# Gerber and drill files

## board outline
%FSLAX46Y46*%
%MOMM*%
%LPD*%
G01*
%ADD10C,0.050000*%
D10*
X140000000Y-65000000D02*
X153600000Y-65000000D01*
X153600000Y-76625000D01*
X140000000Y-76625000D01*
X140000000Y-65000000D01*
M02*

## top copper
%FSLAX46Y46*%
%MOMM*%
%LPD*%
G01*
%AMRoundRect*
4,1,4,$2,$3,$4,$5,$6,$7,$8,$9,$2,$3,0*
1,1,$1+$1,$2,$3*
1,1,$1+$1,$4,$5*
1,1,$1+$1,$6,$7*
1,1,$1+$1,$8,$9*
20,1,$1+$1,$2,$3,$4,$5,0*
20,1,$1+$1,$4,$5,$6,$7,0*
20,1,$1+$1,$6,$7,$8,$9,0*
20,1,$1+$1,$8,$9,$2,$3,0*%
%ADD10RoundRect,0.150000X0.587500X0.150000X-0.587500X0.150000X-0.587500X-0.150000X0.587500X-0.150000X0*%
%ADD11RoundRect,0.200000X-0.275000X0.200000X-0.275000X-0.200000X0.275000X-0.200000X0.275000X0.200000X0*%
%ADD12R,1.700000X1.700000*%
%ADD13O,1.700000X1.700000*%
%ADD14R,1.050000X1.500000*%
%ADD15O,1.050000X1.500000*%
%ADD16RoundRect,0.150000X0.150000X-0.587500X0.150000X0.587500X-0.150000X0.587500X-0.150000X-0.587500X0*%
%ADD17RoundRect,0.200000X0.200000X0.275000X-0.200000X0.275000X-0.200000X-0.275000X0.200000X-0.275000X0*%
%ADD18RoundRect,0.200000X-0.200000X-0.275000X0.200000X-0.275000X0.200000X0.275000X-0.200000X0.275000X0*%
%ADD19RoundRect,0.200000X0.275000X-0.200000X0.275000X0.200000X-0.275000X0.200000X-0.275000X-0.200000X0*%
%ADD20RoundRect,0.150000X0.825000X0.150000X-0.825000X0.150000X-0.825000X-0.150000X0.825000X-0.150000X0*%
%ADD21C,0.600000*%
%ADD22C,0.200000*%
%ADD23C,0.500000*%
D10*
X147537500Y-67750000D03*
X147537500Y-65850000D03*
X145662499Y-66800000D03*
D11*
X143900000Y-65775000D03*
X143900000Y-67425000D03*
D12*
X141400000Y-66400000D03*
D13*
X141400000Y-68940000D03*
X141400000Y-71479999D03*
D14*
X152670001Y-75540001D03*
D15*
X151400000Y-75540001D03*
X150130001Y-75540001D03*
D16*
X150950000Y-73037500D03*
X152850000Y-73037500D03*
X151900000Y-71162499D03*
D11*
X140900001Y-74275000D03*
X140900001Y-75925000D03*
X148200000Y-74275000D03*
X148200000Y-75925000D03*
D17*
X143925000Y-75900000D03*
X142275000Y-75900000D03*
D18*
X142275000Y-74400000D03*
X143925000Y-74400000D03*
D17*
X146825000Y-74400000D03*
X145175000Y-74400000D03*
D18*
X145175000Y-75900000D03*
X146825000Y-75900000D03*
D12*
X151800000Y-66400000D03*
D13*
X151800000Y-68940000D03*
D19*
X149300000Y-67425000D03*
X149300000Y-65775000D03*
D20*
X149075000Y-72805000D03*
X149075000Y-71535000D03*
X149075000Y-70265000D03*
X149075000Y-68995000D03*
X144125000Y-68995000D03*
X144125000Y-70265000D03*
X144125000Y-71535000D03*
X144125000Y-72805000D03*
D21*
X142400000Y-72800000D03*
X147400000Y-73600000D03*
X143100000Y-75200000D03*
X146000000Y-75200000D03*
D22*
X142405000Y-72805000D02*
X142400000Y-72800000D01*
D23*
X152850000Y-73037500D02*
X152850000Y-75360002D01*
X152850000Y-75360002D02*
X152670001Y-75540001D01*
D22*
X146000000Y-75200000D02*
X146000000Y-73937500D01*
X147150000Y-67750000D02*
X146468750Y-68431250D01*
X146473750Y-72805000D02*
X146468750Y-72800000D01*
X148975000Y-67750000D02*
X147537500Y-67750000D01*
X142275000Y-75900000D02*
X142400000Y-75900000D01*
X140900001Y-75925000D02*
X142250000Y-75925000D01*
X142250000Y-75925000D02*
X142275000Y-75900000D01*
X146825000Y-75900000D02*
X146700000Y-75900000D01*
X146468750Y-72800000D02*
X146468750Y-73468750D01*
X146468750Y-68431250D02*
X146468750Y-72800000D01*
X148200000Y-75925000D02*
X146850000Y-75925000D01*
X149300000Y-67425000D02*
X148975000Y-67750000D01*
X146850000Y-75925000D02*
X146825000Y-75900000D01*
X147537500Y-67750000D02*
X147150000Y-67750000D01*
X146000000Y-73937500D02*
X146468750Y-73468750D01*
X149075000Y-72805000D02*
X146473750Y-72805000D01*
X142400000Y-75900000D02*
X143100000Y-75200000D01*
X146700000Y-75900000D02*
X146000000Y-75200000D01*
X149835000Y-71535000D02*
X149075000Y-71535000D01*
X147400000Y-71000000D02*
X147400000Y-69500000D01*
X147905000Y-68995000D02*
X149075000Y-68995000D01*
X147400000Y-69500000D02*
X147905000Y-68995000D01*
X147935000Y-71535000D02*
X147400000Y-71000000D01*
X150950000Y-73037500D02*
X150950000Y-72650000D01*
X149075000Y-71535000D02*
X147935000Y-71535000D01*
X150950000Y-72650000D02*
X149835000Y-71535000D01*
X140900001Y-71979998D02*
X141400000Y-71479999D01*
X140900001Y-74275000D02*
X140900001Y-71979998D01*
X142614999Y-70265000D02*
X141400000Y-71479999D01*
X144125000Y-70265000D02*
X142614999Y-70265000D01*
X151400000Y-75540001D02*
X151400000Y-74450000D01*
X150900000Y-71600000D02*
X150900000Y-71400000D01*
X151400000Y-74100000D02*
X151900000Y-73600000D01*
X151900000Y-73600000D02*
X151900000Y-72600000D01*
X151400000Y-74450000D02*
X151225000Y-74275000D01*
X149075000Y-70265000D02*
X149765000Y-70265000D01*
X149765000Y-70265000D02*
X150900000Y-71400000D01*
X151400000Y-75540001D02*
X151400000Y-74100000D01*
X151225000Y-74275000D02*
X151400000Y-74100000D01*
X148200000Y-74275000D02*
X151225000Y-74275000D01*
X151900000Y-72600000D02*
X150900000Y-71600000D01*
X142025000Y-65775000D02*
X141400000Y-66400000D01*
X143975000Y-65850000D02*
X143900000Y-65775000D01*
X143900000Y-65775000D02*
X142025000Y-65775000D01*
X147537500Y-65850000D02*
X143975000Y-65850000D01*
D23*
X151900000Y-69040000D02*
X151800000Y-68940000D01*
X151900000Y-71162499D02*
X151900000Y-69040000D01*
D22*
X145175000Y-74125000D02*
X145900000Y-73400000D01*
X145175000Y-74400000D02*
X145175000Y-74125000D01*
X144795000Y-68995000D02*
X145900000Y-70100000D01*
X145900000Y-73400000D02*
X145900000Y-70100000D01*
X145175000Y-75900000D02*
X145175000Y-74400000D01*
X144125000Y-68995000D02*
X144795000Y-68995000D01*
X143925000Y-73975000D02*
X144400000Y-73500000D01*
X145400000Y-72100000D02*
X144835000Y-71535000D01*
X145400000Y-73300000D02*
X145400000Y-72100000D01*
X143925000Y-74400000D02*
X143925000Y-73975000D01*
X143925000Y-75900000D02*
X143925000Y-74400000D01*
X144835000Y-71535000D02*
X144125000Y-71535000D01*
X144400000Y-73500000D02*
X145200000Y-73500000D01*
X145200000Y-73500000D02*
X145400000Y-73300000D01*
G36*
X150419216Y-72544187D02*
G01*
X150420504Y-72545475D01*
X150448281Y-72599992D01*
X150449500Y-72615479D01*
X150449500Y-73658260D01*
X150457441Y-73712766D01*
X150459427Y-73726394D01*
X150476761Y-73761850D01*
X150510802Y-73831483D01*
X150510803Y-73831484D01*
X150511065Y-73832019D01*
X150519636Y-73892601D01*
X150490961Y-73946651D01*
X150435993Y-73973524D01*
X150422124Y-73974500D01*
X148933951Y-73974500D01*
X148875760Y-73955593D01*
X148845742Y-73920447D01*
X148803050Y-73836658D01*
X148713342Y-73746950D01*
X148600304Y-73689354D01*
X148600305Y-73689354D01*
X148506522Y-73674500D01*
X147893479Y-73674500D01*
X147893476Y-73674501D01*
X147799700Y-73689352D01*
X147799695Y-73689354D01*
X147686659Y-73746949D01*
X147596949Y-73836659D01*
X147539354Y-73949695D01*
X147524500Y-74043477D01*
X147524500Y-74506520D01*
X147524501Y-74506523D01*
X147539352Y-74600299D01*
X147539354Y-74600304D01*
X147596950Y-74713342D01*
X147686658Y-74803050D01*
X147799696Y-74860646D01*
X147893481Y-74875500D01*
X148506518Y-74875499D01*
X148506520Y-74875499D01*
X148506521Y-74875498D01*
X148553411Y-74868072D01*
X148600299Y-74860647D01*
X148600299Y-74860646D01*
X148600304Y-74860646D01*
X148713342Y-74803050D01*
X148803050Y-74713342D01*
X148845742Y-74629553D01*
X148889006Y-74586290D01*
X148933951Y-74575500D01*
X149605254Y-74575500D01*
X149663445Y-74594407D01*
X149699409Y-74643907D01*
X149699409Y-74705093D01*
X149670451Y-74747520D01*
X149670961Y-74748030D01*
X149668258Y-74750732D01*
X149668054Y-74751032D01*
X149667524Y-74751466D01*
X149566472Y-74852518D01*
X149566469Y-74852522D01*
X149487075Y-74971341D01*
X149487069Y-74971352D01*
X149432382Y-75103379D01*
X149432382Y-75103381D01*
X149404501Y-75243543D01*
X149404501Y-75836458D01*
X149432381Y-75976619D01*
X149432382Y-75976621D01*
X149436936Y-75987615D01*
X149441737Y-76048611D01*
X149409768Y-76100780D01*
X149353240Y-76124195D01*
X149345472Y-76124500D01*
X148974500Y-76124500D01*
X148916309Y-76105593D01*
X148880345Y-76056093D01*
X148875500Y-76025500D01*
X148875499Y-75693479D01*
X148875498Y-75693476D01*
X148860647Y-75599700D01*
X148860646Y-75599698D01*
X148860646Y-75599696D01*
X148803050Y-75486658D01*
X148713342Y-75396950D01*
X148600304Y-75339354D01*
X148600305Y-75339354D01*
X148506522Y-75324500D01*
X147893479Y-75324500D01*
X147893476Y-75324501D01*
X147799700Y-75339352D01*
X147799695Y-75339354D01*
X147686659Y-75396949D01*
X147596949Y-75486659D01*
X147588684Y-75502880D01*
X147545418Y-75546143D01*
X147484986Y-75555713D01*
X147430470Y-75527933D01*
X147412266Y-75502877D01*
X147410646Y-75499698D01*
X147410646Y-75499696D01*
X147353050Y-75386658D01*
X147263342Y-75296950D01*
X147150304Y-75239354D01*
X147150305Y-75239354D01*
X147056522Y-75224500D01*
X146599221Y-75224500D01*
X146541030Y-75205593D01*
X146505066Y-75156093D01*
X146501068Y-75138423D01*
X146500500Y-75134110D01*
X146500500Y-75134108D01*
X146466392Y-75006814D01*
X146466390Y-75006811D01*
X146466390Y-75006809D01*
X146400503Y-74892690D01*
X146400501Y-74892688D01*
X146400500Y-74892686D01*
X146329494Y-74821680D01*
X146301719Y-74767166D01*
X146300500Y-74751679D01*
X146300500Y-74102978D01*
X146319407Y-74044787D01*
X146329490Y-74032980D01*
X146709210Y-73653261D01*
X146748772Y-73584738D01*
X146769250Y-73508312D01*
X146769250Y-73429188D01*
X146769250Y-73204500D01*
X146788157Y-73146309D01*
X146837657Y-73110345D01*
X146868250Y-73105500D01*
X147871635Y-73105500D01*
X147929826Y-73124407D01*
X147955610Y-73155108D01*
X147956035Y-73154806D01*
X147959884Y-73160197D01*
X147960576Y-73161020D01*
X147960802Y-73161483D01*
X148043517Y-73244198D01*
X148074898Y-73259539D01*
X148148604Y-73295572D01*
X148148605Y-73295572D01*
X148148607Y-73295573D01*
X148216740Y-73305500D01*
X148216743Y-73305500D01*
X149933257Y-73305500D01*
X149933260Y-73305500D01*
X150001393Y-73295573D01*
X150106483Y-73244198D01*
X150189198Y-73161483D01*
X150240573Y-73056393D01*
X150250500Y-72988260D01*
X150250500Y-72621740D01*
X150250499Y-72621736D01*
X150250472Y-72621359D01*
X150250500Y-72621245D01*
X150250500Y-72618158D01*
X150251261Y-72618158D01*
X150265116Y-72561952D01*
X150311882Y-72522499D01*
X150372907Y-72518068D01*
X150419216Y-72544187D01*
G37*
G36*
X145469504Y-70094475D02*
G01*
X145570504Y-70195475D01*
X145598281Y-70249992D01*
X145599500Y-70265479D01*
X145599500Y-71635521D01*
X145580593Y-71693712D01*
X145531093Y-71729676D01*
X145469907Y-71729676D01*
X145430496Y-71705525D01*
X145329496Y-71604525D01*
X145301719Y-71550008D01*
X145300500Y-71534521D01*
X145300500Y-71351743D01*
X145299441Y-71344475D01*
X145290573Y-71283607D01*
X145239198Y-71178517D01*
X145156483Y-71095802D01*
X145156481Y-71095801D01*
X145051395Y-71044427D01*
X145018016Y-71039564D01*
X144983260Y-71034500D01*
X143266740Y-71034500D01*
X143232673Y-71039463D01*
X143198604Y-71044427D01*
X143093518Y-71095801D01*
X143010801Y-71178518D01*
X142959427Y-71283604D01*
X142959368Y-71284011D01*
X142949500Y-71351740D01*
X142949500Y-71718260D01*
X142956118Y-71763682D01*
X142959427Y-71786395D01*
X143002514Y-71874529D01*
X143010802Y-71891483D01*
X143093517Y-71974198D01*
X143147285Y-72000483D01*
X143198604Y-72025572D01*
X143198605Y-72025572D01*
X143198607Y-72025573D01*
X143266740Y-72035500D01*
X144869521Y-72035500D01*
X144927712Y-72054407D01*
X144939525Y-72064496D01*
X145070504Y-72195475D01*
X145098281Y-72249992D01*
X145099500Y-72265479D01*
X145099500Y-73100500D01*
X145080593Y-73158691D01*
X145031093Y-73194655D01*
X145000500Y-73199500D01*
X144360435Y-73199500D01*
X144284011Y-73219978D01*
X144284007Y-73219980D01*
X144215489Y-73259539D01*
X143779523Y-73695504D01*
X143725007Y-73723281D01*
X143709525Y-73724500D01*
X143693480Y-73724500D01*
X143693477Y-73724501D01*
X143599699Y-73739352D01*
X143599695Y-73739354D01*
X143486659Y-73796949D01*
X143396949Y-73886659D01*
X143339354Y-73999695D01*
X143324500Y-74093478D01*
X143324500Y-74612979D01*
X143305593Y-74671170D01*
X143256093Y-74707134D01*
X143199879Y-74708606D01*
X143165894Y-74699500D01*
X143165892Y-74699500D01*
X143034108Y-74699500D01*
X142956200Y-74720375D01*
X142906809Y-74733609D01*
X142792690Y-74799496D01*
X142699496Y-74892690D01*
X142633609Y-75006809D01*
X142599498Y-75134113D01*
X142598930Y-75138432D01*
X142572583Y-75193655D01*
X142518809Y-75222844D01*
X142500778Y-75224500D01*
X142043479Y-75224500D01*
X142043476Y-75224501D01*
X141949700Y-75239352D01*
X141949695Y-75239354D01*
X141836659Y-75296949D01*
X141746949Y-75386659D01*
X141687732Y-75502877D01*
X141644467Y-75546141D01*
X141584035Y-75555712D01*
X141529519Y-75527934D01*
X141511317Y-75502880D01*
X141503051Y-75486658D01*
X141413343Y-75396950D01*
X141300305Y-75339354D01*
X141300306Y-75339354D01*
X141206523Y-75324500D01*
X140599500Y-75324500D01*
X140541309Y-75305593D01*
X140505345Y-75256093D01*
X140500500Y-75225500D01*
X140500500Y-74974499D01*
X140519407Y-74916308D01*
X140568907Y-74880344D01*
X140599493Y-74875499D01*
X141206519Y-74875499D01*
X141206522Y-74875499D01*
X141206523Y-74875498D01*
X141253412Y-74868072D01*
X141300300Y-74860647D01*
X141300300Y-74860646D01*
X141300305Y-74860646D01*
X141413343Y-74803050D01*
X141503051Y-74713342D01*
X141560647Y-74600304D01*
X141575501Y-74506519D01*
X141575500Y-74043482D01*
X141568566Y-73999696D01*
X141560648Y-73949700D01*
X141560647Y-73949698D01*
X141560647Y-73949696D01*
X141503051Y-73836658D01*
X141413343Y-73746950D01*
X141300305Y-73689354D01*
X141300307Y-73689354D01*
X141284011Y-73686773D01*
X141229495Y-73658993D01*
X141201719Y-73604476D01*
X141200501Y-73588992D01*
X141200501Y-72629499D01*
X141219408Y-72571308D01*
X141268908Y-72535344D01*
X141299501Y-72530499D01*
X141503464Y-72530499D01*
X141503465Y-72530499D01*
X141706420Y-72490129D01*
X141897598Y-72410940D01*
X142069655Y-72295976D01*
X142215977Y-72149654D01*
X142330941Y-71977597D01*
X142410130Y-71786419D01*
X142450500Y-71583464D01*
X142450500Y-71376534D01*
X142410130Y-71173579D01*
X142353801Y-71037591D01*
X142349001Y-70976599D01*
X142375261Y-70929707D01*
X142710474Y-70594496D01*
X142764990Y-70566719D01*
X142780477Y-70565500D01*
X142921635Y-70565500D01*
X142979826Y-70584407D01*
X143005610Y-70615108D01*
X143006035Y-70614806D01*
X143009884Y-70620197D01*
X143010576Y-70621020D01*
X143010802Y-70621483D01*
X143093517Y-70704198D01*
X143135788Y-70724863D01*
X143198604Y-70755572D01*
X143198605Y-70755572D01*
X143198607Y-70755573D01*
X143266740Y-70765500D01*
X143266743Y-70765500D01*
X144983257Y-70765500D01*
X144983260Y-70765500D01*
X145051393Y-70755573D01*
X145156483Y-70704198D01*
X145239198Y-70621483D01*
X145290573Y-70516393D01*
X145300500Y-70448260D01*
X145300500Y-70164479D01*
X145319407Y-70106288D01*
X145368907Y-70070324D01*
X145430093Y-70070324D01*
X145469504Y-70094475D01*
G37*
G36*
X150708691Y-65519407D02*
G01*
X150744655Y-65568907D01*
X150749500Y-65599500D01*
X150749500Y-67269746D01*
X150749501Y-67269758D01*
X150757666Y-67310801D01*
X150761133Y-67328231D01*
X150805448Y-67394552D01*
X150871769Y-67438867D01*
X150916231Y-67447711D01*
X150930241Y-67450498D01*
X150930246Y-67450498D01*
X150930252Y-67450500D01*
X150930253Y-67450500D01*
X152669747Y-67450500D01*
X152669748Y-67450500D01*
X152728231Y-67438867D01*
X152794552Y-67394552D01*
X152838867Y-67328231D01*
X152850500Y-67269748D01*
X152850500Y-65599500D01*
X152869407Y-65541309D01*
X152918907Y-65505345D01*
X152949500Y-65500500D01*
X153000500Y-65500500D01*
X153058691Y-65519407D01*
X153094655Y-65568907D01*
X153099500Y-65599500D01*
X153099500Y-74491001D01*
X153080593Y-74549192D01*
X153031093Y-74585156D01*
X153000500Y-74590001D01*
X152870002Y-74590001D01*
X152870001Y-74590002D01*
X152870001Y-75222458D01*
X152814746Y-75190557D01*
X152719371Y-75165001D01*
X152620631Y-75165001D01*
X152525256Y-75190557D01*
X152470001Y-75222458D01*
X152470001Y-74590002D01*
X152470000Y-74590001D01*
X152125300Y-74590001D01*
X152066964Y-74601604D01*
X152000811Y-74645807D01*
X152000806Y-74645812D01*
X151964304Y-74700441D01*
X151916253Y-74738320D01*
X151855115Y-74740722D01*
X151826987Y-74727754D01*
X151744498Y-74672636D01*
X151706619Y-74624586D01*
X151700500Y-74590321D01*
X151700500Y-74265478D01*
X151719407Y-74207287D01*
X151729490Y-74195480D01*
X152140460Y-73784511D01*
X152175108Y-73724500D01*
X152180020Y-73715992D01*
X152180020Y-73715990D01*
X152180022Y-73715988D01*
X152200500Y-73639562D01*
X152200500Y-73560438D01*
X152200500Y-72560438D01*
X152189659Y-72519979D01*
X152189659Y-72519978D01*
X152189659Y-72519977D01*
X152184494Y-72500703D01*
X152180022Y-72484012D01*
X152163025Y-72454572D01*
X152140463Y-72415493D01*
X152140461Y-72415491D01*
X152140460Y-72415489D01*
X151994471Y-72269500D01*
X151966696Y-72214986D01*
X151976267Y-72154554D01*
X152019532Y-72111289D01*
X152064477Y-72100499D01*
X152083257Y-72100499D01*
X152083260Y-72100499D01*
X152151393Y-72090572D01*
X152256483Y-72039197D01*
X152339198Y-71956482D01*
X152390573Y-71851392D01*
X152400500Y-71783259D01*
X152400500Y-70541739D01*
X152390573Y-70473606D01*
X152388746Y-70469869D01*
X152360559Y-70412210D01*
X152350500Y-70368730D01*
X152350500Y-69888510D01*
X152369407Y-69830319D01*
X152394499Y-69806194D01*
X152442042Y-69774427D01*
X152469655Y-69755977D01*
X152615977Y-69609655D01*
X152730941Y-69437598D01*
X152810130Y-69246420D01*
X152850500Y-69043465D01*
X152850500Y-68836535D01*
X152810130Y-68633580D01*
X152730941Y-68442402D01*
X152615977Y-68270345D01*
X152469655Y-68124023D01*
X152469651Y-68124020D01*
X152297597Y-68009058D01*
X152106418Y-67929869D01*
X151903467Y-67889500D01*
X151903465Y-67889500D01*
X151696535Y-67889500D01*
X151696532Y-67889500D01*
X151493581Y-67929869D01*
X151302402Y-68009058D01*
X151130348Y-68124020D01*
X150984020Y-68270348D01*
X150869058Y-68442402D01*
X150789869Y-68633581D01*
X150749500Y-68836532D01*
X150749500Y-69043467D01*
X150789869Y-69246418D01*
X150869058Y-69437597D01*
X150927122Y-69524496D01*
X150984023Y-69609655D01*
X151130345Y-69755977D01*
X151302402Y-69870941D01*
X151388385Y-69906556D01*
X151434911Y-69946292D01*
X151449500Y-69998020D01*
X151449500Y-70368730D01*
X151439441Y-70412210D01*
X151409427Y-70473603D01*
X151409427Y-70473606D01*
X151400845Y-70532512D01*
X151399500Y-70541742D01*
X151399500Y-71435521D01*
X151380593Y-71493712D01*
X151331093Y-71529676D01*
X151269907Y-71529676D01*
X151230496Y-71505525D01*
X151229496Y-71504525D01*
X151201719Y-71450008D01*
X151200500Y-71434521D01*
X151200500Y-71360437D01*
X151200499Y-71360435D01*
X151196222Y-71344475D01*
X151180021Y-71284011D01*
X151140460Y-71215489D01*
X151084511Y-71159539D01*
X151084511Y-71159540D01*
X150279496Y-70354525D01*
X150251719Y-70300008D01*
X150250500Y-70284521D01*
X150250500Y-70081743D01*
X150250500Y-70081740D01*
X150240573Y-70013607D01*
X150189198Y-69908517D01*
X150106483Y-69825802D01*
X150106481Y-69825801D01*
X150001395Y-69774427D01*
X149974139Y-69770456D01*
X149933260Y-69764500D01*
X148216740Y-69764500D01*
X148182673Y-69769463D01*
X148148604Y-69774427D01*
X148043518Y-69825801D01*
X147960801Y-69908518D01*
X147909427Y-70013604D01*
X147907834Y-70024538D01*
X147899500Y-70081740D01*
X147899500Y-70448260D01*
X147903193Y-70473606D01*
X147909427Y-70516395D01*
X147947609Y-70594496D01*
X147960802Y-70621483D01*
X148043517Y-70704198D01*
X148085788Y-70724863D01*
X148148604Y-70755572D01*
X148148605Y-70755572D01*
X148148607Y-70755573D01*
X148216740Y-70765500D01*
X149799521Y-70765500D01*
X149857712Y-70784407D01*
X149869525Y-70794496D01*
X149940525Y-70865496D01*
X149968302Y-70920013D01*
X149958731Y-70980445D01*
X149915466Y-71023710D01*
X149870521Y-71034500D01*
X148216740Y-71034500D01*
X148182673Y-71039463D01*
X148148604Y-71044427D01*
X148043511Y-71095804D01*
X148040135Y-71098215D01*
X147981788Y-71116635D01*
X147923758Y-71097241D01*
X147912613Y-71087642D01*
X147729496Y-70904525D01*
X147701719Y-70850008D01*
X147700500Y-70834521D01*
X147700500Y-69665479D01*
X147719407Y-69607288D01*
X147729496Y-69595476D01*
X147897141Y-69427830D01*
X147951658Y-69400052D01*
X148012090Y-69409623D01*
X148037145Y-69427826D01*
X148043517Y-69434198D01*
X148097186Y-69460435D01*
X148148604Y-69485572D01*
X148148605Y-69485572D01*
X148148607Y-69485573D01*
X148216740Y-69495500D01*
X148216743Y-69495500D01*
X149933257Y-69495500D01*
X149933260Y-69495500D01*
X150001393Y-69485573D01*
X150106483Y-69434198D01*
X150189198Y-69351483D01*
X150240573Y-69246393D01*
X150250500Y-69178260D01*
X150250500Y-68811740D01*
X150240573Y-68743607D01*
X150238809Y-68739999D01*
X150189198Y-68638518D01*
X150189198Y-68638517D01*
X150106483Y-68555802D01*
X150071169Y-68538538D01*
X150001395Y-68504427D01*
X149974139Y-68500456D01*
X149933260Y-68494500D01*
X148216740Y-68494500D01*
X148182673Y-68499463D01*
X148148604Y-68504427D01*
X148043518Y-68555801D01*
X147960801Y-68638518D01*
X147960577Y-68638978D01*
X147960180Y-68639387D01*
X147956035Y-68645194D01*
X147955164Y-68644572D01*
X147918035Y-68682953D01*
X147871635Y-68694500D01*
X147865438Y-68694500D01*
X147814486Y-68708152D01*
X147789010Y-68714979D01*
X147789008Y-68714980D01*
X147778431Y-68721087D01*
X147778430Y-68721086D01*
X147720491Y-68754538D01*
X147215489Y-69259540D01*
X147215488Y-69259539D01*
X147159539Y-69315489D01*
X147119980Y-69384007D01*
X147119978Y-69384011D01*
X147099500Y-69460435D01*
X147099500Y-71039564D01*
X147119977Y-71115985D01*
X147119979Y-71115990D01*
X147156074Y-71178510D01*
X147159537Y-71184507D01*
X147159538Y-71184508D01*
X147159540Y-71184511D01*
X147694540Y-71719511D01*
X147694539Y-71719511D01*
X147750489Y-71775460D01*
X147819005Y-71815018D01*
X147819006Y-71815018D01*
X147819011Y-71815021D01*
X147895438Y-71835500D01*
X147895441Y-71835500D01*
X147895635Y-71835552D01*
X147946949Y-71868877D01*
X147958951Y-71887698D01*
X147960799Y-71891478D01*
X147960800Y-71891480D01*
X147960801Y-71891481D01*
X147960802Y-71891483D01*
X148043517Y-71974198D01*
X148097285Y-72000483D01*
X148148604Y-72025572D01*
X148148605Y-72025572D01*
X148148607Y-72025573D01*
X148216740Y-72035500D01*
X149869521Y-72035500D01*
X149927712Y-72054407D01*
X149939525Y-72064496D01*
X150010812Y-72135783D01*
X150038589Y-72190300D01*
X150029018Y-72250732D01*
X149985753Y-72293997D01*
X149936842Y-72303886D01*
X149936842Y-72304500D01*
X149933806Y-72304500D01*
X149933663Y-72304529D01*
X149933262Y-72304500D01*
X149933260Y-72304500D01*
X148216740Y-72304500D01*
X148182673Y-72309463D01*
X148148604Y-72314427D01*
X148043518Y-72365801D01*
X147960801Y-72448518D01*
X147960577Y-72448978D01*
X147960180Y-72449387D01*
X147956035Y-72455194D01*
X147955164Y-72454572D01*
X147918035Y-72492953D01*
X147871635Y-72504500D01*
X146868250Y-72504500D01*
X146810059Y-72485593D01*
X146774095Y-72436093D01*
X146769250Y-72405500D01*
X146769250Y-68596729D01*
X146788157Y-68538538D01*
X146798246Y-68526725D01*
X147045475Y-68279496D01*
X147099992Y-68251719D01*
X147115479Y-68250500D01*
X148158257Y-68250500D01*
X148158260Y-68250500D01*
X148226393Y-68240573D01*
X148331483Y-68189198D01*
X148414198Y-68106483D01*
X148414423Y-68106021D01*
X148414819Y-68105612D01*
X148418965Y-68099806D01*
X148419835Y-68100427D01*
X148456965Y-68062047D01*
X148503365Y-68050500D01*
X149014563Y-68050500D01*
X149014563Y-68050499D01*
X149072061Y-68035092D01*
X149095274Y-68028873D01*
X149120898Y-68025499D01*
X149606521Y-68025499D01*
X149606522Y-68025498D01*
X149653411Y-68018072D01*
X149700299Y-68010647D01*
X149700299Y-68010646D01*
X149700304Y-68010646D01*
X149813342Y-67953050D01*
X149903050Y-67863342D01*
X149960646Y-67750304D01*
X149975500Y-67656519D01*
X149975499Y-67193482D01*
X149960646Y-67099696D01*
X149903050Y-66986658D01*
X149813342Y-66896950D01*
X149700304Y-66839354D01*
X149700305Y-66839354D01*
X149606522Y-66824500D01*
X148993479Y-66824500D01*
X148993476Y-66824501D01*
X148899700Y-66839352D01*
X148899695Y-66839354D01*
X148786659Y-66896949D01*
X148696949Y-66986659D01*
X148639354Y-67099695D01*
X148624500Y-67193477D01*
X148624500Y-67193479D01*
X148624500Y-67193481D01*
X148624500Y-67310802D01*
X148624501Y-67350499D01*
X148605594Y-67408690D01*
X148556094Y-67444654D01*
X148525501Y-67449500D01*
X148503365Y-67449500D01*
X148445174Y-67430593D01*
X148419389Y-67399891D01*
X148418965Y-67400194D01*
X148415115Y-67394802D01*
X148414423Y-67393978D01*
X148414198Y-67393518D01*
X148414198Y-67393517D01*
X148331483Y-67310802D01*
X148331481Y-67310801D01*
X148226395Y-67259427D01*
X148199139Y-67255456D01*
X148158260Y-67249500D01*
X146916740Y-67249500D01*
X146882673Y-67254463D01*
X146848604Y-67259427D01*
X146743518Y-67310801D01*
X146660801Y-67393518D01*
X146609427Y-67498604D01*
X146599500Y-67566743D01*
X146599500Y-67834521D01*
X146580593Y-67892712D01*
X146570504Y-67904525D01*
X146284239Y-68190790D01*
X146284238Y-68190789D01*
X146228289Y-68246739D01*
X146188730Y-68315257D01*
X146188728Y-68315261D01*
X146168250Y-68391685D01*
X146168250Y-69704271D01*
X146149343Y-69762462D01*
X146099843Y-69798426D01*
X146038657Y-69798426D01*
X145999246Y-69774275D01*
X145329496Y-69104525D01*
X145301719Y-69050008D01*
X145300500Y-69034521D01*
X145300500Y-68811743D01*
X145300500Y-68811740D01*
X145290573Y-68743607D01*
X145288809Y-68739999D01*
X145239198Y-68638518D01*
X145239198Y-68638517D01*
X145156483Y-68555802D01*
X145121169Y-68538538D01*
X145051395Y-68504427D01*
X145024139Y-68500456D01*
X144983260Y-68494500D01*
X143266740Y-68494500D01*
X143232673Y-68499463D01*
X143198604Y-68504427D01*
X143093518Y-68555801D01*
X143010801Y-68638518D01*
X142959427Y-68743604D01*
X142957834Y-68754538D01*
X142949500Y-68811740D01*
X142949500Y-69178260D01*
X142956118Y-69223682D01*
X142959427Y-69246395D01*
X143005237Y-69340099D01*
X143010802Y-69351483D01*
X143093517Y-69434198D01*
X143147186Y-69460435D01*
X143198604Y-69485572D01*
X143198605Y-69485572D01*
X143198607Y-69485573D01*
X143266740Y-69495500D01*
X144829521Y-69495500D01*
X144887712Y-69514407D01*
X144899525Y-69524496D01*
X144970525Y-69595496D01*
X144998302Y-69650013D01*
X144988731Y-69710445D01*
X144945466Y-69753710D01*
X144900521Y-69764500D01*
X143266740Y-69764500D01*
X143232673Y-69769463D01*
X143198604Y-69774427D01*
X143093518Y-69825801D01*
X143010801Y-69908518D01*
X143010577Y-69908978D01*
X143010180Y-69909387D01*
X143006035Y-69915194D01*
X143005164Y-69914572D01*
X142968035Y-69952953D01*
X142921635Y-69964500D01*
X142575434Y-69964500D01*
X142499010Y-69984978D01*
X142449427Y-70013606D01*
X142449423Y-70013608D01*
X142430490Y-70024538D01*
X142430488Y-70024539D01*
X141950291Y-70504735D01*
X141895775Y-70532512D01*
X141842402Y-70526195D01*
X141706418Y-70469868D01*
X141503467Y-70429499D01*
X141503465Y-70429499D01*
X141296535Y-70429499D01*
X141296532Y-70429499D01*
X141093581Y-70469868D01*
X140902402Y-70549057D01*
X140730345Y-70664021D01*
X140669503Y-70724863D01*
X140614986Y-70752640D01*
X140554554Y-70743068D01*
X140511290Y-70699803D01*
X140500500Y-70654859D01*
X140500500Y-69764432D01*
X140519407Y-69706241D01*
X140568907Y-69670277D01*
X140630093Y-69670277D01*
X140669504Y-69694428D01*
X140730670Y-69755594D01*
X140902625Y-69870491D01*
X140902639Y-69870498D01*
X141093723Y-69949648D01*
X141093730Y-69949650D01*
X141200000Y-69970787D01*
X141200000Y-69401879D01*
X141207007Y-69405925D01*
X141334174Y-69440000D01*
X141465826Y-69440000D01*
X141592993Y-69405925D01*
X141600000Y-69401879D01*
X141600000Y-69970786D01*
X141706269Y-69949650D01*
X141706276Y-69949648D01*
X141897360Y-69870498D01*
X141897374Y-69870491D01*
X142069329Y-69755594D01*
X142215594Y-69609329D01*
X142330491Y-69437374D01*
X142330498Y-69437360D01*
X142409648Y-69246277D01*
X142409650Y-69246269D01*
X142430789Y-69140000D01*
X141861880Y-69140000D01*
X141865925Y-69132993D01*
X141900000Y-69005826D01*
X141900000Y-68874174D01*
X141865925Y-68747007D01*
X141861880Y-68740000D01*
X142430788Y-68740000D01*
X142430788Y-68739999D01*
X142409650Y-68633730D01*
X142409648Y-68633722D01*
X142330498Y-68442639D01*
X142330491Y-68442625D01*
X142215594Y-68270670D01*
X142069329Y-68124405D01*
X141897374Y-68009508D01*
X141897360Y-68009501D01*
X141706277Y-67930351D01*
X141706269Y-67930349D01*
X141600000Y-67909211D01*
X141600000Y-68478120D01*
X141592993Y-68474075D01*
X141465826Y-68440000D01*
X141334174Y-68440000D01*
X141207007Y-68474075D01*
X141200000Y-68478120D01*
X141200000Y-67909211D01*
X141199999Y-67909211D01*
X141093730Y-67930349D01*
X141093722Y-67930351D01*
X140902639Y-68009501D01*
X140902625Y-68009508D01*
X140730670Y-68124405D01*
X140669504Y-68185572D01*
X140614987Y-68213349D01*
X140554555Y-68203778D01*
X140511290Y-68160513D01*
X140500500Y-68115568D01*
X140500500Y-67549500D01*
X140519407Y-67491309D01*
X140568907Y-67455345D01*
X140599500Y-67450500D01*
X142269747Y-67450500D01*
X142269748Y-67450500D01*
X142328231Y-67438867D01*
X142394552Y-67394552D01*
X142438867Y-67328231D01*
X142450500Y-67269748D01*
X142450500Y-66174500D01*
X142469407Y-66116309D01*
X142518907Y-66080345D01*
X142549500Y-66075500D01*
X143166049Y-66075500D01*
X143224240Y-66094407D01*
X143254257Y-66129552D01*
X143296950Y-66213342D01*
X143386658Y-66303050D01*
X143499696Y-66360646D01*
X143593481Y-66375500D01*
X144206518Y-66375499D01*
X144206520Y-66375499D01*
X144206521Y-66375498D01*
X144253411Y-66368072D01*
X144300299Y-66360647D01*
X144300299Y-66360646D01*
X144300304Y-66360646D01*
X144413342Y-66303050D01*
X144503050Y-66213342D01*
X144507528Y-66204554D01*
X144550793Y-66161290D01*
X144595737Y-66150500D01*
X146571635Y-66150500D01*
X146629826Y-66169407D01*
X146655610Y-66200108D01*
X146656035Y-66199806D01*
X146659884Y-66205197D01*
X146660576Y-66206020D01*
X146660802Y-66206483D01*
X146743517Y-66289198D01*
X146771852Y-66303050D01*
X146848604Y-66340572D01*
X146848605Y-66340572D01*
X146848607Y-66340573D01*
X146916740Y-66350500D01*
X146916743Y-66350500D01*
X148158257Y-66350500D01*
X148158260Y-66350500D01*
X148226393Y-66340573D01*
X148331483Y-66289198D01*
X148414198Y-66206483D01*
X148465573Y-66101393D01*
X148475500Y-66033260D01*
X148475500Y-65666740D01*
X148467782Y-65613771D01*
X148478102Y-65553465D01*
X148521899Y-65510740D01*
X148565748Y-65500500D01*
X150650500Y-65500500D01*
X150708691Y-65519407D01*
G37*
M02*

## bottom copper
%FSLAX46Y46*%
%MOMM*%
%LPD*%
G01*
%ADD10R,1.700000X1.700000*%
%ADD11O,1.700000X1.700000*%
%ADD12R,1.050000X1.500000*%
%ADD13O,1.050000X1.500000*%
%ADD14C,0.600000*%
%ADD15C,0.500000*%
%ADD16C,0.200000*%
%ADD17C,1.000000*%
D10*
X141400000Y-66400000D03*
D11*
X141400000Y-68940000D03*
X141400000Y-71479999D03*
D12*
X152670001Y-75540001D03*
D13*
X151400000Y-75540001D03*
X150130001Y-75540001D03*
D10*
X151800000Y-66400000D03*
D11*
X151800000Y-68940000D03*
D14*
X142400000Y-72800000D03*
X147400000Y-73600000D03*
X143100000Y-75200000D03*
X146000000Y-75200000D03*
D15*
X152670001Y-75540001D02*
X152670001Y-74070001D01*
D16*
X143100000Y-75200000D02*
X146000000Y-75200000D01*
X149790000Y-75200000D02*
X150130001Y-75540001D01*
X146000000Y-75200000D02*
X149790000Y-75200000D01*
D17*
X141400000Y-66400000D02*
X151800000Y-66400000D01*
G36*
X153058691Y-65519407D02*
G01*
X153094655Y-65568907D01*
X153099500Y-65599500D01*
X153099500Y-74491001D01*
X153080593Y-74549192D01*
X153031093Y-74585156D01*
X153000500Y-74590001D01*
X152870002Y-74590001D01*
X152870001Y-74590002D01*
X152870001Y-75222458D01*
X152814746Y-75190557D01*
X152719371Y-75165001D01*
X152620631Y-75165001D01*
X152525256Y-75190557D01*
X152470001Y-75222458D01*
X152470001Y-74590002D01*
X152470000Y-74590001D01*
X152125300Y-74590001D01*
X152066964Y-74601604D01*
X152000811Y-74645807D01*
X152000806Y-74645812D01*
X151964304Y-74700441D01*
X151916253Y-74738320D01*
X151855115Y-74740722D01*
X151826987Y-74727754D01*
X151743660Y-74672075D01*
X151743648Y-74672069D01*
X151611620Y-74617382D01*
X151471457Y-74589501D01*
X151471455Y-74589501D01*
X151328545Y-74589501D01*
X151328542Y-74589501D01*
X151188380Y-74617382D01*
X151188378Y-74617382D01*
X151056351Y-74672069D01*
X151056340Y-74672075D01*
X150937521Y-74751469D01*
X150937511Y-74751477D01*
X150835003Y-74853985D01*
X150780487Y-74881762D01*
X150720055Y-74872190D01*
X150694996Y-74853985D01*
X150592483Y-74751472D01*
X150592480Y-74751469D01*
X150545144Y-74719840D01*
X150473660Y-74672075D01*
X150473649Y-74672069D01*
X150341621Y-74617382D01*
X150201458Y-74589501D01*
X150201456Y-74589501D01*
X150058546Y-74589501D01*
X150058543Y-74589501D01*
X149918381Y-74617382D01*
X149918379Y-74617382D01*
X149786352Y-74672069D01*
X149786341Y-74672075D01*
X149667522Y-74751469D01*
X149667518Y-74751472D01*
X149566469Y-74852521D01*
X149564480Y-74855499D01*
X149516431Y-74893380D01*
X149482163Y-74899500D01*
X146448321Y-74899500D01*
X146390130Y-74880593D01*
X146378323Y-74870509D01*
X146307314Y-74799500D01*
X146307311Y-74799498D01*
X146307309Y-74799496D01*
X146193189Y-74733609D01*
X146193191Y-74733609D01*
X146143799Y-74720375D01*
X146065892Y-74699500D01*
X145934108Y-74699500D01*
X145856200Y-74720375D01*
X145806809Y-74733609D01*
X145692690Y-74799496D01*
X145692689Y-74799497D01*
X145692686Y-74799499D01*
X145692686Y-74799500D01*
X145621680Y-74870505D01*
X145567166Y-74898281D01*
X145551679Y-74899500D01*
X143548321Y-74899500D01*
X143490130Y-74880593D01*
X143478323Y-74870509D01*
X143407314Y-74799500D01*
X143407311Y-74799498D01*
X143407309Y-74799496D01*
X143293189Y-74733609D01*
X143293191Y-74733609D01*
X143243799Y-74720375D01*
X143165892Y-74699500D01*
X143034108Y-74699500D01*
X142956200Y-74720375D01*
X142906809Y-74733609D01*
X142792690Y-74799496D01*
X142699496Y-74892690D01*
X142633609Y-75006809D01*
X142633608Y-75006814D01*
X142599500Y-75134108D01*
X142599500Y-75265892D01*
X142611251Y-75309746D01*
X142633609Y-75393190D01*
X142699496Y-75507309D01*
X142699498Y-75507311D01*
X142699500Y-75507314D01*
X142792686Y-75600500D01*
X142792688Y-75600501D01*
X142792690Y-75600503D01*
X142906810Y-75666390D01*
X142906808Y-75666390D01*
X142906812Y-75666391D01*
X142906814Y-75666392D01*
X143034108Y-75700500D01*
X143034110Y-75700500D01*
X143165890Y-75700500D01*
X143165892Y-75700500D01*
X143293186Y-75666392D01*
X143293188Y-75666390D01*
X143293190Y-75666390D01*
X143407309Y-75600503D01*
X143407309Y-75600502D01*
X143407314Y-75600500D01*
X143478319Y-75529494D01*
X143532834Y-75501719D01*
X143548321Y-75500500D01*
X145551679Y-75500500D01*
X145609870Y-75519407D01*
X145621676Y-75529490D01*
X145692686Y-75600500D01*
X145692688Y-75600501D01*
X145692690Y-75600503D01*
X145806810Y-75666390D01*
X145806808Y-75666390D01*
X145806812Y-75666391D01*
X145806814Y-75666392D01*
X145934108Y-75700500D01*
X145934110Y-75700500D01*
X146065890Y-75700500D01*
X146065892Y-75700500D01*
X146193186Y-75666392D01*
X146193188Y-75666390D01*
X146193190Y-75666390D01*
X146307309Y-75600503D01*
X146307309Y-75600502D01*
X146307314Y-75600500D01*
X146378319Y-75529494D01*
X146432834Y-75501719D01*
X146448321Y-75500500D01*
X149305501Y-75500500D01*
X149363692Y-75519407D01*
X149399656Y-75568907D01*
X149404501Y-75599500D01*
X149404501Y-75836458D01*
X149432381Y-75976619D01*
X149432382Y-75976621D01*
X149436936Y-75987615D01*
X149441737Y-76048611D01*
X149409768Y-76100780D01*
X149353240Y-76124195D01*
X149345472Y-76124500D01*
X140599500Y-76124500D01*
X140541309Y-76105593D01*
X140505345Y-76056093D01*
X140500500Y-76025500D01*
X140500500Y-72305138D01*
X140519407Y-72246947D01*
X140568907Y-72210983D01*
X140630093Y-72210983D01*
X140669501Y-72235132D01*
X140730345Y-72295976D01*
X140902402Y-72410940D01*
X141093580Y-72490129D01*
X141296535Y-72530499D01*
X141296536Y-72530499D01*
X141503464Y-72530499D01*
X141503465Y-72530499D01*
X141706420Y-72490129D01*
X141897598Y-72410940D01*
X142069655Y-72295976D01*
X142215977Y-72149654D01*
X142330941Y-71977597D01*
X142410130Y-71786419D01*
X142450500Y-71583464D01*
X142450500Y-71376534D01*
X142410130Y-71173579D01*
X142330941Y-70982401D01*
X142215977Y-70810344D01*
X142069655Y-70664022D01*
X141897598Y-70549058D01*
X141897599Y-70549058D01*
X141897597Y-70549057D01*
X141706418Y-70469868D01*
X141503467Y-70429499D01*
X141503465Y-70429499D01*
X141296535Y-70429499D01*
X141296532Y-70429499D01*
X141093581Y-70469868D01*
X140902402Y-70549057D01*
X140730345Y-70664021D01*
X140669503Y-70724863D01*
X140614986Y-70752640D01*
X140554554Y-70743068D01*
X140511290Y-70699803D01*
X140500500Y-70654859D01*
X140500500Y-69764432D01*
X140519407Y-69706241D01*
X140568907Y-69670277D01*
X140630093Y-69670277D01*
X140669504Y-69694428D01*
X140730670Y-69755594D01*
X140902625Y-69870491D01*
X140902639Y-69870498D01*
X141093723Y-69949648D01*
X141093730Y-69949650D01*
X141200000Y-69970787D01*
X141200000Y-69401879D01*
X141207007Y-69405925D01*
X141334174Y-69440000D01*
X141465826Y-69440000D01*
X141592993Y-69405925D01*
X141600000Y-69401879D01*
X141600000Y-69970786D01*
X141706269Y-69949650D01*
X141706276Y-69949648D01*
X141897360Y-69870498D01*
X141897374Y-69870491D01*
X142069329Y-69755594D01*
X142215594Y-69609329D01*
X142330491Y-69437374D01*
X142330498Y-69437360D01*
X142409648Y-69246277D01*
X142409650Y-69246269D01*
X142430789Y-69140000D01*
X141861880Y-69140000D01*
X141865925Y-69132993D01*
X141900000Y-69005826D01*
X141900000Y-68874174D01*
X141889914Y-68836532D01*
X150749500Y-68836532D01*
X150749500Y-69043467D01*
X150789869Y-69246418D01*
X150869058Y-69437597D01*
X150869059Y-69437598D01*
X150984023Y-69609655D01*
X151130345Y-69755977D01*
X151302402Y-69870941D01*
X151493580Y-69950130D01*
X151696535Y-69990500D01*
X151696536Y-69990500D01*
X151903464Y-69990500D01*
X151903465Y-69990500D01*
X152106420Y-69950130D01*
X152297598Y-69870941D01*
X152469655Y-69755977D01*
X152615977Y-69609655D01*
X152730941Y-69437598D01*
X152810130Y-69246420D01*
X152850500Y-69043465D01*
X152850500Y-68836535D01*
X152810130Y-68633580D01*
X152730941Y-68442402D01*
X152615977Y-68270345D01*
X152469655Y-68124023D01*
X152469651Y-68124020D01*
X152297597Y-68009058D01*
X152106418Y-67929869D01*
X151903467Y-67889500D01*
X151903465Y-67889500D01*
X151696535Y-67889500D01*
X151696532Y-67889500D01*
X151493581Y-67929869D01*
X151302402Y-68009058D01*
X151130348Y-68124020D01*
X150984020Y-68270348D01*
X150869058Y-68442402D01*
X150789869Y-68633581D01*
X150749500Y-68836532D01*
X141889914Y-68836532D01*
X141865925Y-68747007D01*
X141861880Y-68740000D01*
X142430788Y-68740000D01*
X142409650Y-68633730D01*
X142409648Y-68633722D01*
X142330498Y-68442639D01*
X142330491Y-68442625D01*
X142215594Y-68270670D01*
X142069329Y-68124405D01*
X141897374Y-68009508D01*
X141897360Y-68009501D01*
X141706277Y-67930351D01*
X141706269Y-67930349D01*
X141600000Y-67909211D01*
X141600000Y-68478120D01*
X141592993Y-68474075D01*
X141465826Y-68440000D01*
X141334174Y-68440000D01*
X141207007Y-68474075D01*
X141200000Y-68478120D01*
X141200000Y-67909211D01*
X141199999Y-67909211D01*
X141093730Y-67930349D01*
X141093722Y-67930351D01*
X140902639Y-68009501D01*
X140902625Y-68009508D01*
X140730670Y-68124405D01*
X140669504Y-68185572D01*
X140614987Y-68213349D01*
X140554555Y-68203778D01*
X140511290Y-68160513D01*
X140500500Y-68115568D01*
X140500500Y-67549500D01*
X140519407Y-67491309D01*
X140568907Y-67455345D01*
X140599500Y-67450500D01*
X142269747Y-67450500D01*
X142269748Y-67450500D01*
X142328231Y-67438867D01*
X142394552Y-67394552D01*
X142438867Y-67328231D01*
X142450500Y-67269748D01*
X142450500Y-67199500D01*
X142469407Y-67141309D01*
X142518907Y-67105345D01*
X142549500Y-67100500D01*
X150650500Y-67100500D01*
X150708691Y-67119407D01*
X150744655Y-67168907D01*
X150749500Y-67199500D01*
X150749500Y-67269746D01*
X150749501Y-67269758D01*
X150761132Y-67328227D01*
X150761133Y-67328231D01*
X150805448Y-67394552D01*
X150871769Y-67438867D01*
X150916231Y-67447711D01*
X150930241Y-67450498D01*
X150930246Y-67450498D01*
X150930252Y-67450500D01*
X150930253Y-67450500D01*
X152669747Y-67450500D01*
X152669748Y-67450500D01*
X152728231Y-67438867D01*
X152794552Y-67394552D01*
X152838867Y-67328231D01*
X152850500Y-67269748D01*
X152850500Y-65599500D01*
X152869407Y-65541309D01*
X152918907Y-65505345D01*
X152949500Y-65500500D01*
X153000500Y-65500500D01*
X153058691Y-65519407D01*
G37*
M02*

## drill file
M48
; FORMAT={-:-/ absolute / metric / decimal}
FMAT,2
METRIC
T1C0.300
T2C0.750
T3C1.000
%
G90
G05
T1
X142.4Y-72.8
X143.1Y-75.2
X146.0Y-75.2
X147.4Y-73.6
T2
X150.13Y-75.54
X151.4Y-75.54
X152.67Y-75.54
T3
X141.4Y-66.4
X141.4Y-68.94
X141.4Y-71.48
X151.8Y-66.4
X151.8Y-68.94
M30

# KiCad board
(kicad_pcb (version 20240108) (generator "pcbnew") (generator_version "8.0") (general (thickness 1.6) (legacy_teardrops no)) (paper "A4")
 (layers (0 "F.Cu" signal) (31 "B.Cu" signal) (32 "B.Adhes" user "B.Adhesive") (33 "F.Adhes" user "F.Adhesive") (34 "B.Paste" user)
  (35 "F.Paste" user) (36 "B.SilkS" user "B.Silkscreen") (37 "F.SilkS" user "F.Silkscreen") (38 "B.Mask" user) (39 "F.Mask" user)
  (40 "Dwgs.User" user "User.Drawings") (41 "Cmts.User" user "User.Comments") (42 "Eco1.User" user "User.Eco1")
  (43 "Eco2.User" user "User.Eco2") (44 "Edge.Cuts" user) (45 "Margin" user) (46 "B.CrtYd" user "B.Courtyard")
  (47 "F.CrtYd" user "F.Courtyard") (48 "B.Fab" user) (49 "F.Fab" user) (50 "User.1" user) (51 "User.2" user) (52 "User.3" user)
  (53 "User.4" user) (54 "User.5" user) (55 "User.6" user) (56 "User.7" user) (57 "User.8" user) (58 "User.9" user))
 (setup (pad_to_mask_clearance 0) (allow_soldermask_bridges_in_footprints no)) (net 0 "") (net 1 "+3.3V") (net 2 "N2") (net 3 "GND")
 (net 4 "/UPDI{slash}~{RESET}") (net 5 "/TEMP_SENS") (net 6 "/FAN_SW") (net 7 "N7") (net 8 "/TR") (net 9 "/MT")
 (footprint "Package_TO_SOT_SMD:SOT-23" (layer "F.Cu") (at 146.6 66.8 180)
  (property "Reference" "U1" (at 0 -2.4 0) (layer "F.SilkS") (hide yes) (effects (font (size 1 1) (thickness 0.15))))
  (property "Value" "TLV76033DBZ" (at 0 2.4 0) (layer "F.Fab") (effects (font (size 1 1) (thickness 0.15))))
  (pad "1" smd roundrect (at -0.9375 -0.95 180) (size 1.475 0.6) (layers "F.Cu" "F.Paste" "F.Mask") (roundrect_rratio 0.25) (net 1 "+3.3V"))
  (pad "2" smd roundrect (at -0.9375 0.95 180) (size 1.475 0.6) (layers "F.Cu" "F.Paste" "F.Mask") (roundrect_rratio 0.25) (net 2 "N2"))
  (pad "3" smd roundrect (at 0.937501 0 180) (size 1.475 0.6) (layers "F.Cu" "F.Paste" "F.Mask") (roundrect_rratio 0.25) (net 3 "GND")))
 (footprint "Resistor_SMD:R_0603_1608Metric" (layer "F.Cu") (at 143.9 66.6 -90)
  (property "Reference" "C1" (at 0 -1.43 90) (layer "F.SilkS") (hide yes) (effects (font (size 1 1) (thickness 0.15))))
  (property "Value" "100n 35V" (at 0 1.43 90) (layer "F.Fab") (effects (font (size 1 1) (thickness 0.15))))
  (pad "1" smd roundrect (at -0.825 0 270) (size 0.8 0.95) (layers "F.Cu" "F.Paste" "F.Mask") (roundrect_rratio 0.25) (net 2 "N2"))
  (pad "2" smd roundrect (at 0.825 0 270) (size 0.8 0.95) (layers "F.Cu" "F.Paste" "F.Mask") (roundrect_rratio 0.25) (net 3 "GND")))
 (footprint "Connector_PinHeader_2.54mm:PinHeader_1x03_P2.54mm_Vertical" (layer "F.Cu") (at 141.4 66.4)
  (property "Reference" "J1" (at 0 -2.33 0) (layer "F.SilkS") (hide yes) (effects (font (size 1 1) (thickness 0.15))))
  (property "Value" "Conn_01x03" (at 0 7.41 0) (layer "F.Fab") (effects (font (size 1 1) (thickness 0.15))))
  (pad "1" thru_hole rect (at 0 0) (size 1.7 1.7) (drill 1) (layers "*.Cu" "*.Mask") (remove_unused_layers no) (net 2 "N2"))
  (pad "2" thru_hole oval (at 0 2.54) (size 1.7 1.7) (drill 1) (layers "*.Cu" "*.Mask") (remove_unused_layers no) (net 3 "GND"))
  (pad "3" thru_hole oval (at 0 5.079999) (size 1.7 1.7) (drill 1) (layers "*.Cu" "*.Mask") (remove_unused_layers no)
   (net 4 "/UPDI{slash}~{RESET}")))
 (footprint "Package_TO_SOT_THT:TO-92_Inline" (layer "F.Cu") (at 152.670001 75.540001 180)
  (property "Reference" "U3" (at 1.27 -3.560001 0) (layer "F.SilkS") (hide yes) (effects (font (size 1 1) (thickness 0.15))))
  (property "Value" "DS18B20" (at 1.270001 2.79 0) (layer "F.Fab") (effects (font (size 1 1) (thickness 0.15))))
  (pad "1" thru_hole rect (at 0 0 180) (size 1.05 1.5) (drill 0.75) (layers "*.Cu" "*.Mask") (remove_unused_layers no) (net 3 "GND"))
  (pad "2" thru_hole oval (at 1.270001 0 180) (size 1.05 1.5) (drill 0.75) (layers "*.Cu" "*.Mask") (remove_unused_layers no)
   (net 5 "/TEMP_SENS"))
  (pad "3" thru_hole oval (at 2.54 0 180) (size 1.05 1.5) (drill 0.75) (layers "*.Cu" "*.Mask") (remove_unused_layers no) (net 1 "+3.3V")))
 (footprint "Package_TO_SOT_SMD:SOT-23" (layer "F.Cu") (at 151.9 72.1 90)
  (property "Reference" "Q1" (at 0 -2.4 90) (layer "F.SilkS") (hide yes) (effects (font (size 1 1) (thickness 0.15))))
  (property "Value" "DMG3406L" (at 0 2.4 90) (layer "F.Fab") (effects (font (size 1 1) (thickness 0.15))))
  (pad "1" smd roundrect (at -0.9375 -0.95 90) (size 1.475 0.6) (layers "F.Cu" "F.Paste" "F.Mask") (roundrect_rratio 0.25) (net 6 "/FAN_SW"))
  (pad "2" smd roundrect (at -0.9375 0.95 90) (size 1.475 0.6) (layers "F.Cu" "F.Paste" "F.Mask") (roundrect_rratio 0.25) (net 3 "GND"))
  (pad "3" smd roundrect (at 0.937501 0 90) (size 1.475 0.6) (layers "F.Cu" "F.Paste" "F.Mask") (roundrect_rratio 0.25) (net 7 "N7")))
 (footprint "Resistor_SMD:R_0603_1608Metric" (layer "F.Cu") (at 140.900001 75.1 -90)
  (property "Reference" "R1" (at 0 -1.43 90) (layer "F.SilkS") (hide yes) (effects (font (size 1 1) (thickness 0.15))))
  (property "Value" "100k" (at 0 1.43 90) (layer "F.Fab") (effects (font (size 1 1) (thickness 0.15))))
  (pad "1" smd roundrect (at -0.825 0 270) (size 0.8 0.95) (layers "F.Cu" "F.Paste" "F.Mask") (roundrect_rratio 0.25)
   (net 4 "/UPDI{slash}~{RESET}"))
  (pad "2" smd roundrect (at 0.825 0 270) (size 0.8 0.95) (layers "F.Cu" "F.Paste" "F.Mask") (roundrect_rratio 0.25) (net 1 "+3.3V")))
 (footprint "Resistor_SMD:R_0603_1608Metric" (layer "F.Cu") (at 148.2 75.1 -90)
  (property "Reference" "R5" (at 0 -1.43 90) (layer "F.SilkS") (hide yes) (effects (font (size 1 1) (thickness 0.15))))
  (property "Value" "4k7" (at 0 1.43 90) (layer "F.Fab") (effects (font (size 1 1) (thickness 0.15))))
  (pad "1" smd roundrect (at -0.825 0 270) (size 0.8 0.95) (layers "F.Cu" "F.Paste" "F.Mask") (roundrect_rratio 0.25) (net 5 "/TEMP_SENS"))
  (pad "2" smd roundrect (at 0.825 0 270) (size 0.8 0.95) (layers "F.Cu" "F.Paste" "F.Mask") (roundrect_rratio 0.25) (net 1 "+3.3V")))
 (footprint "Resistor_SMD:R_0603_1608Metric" (layer "F.Cu") (at 143.1 75.9 180)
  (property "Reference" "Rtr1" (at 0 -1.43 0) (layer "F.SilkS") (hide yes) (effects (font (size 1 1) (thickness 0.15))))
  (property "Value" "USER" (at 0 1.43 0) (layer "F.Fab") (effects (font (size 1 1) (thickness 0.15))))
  (pad "1" smd roundrect (at -0.825 0 180) (size 0.8 0.95) (layers "F.Cu" "F.Paste" "F.Mask") (roundrect_rratio 0.25) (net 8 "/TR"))
  (pad "2" smd roundrect (at 0.825 0 180) (size 0.8 0.95) (layers "F.Cu" "F.Paste" "F.Mask") (roundrect_rratio 0.25) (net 1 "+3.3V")))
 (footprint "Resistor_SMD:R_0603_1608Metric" (layer "F.Cu") (at 143.1 74.4)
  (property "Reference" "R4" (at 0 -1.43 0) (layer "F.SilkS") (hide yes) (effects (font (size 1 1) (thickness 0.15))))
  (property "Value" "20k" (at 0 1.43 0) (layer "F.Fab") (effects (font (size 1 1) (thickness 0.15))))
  (pad "1" smd roundrect (at -0.825 0) (size 0.8 0.95) (layers "F.Cu" "F.Paste" "F.Mask") (roundrect_rratio 0.25) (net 3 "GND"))
  (pad "2" smd roundrect (at 0.825 0) (size 0.8 0.95) (layers "F.Cu" "F.Paste" "F.Mask") (roundrect_rratio 0.25) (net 8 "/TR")))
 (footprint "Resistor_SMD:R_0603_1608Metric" (layer "F.Cu") (at 146 74.4 180)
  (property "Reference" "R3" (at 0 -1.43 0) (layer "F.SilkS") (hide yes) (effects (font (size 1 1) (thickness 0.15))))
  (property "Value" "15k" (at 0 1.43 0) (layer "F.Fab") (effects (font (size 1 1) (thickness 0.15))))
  (pad "1" smd roundrect (at -0.825 0 180) (size 0.8 0.95) (layers "F.Cu" "F.Paste" "F.Mask") (roundrect_rratio 0.25) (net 3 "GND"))
  (pad "2" smd roundrect (at 0.825 0 180) (size 0.8 0.95) (layers "F.Cu" "F.Paste" "F.Mask") (roundrect_rratio 0.25) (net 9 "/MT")))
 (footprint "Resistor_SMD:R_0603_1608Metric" (layer "F.Cu") (at 146 75.9)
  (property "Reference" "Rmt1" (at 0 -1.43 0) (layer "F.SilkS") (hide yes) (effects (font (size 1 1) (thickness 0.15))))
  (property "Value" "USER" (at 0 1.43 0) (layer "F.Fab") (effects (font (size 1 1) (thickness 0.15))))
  (pad "1" smd roundrect (at -0.825 0) (size 0.8 0.95) (layers "F.Cu" "F.Paste" "F.Mask") (roundrect_rratio 0.25) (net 9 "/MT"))
  (pad "2" smd roundrect (at 0.825 0) (size 0.8 0.95) (layers "F.Cu" "F.Paste" "F.Mask") (roundrect_rratio 0.25) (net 1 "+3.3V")))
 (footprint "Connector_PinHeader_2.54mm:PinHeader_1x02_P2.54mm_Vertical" (layer "F.Cu") (at 151.8 66.4)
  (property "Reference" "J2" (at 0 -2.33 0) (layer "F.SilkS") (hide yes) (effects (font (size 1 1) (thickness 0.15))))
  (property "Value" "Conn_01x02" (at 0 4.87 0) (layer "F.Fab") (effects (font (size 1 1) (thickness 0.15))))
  (pad "1" thru_hole rect (at 0 0) (size 1.7 1.7) (drill 1) (layers "*.Cu" "*.Mask") (remove_unused_layers no) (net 2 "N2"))
  (pad "2" thru_hole oval (at 0 2.54) (size 1.7 1.7) (drill 1) (layers "*.Cu" "*.Mask") (remove_unused_layers no) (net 7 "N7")))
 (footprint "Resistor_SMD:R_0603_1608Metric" (layer "F.Cu") (at 149.3 66.6 90)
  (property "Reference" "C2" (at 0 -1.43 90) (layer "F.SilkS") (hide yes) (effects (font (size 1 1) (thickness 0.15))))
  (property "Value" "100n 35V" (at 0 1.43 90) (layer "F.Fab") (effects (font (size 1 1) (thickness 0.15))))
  (pad "1" smd roundrect (at -0.825 0 90) (size 0.8 0.95) (layers "F.Cu" "F.Paste" "F.Mask") (roundrect_rratio 0.25) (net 1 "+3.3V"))
  (pad "2" smd roundrect (at 0.825 0 90) (size 0.8 0.95) (layers "F.Cu" "F.Paste" "F.Mask") (roundrect_rratio 0.25) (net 3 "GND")))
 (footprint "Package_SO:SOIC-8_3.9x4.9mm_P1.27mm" (layer "F.Cu") (at 146.6 70.9 180)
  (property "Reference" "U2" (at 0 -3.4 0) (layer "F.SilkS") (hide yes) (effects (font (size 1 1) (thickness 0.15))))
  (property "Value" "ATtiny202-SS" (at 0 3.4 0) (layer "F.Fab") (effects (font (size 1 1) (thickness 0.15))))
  (pad "1" smd roundrect (at -2.475 -1.905 180) (size 1.95 0.6) (layers "F.Cu" "F.Paste" "F.Mask") (roundrect_rratio 0.25) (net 1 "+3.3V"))
  (pad "2" smd roundrect (at -2.475 -0.635 180) (size 1.95 0.6) (layers "F.Cu" "F.Paste" "F.Mask") (roundrect_rratio 0.25) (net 6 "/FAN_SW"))
  (pad "3" smd roundrect (at -2.475 0.635 180) (size 1.95 0.6) (layers "F.Cu" "F.Paste" "F.Mask") (roundrect_rratio 0.25)
   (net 5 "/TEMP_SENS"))
  (pad "4" smd roundrect (at -2.475 1.905 180) (size 1.95 0.6) (layers "F.Cu" "F.Paste" "F.Mask") (roundrect_rratio 0.25) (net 6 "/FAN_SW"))
  (pad "5" smd roundrect (at 2.475 1.905 180) (size 1.95 0.6) (layers "F.Cu" "F.Paste" "F.Mask") (roundrect_rratio 0.25) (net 9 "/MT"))
  (pad "6" smd roundrect (at 2.475 0.635 180) (size 1.95 0.6) (layers "F.Cu" "F.Paste" "F.Mask") (roundrect_rratio 0.25)
   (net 4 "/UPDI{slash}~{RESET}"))
  (pad "7" smd roundrect (at 2.475 -0.635 180) (size 1.95 0.6) (layers "F.Cu" "F.Paste" "F.Mask") (roundrect_rratio 0.25) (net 8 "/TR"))
  (pad "8" smd roundrect (at 2.475 -1.905 180) (size 1.95 0.6) (layers "F.Cu" "F.Paste" "F.Mask") (roundrect_rratio 0.25) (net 3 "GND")))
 (gr_rect (start 140 65) (end 153.6 76.625) (stroke (width 0.05) (type default)) (fill none) (layer "Edge.Cuts"))
 (segment (start 142.405 72.805) (end 142.4 72.8) (width 0.2) (layer "F.Cu") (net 3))
 (segment (start 152.85 73.0375) (end 152.85 75.360002) (width 0.5) (layer "F.Cu") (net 3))
 (segment (start 152.85 75.360002) (end 152.670001 75.540001) (width 0.5) (layer "F.Cu") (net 3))
 (via (at 142.4 72.8) (size 0.6) (drill 0.3) (layers "F.Cu" "B.Cu") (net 3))
 (via (at 147.4 73.6) (size 0.6) (drill 0.3) (layers "F.Cu" "B.Cu") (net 3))
 (segment (start 152.670001 75.540001) (end 152.670001 74.070001) (width 0.5) (layer "B.Cu") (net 3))
 (segment (start 146 75.2) (end 146 73.9375) (width 0.2) (layer "F.Cu") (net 1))
 (segment (start 147.15 67.75) (end 146.46875 68.43125) (width 0.2) (layer "F.Cu") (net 1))
 (segment (start 146.47375 72.805) (end 146.46875 72.8) (width 0.2) (layer "F.Cu") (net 1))
 (segment (start 148.975 67.75) (end 147.5375 67.75) (width 0.2) (layer "F.Cu") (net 1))
 (segment (start 142.275 75.9) (end 142.4 75.9) (width 0.2) (layer "F.Cu") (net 1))
 (segment (start 140.900001 75.925) (end 142.25 75.925) (width 0.2) (layer "F.Cu") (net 1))
 (segment (start 142.25 75.925) (end 142.275 75.9) (width 0.2) (layer "F.Cu") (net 1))
 (segment (start 146.825 75.9) (end 146.7 75.9) (width 0.2) (layer "F.Cu") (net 1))
 (segment (start 146.46875 72.8) (end 146.46875 73.46875) (width 0.2) (layer "F.Cu") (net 1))
 (segment (start 146.46875 68.43125) (end 146.46875 72.8) (width 0.2) (layer "F.Cu") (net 1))
 (segment (start 148.2 75.925) (end 146.85 75.925) (width 0.2) (layer "F.Cu") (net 1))
 (segment (start 149.3 67.425) (end 148.975 67.75) (width 0.2) (layer "F.Cu") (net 1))
 (segment (start 146.85 75.925) (end 146.825 75.9) (width 0.2) (layer "F.Cu") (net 1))
 (segment (start 147.5375 67.75) (end 147.15 67.75) (width 0.2) (layer "F.Cu") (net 1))
 (segment (start 146 73.9375) (end 146.46875 73.46875) (width 0.2) (layer "F.Cu") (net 1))
 (segment (start 149.075 72.805) (end 146.47375 72.805) (width 0.2) (layer "F.Cu") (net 1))
 (segment (start 142.4 75.9) (end 143.1 75.2) (width 0.2) (layer "F.Cu") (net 1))
 (segment (start 146.7 75.9) (end 146 75.2) (width 0.2) (layer "F.Cu") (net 1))
 (via (at 143.1 75.2) (size 0.6) (drill 0.3) (layers "F.Cu" "B.Cu") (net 1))
 (via (at 146 75.2) (size 0.6) (drill 0.3) (layers "F.Cu" "B.Cu") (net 1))
 (segment (start 143.1 75.2) (end 146 75.2) (width 0.2) (layer "B.Cu") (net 1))
 (segment (start 149.79 75.2) (end 150.130001 75.540001) (width 0.2) (layer "B.Cu") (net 1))
 (segment (start 146 75.2) (end 149.79 75.2) (width 0.2) (layer "B.Cu") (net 1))
 (segment (start 149.835 71.535) (end 149.075 71.535) (width 0.2) (layer "F.Cu") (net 6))
 (segment (start 147.4 71) (end 147.4 69.5) (width 0.2) (layer "F.Cu") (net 6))
 (segment (start 147.905 68.995) (end 149.075 68.995) (width 0.2) (layer "F.Cu") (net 6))
 (segment (start 147.4 69.5) (end 147.905 68.995) (width 0.2) (layer "F.Cu") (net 6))
 (segment (start 147.935 71.535) (end 147.4 71) (width 0.2) (layer "F.Cu") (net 6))
 (segment (start 150.95 73.0375) (end 150.95 72.65) (width 0.2) (layer "F.Cu") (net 6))
 (segment (start 149.075 71.535) (end 147.935 71.535) (width 0.2) (layer "F.Cu") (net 6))
 (segment (start 150.95 72.65) (end 149.835 71.535) (width 0.2) (layer "F.Cu") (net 6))
 (segment (start 140.900001 71.979998) (end 141.4 71.479999) (width 0.2) (layer "F.Cu") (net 4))
 (segment (start 140.900001 74.275) (end 140.900001 71.979998) (width 0.2) (layer "F.Cu") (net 4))
 (segment (start 142.614999 70.265) (end 141.4 71.479999) (width 0.2) (layer "F.Cu") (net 4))
 (segment (start 144.125 70.265) (end 142.614999 70.265) (width 0.2) (layer "F.Cu") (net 4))
 (segment (start 151.4 75.540001) (end 151.4 74.45) (width 0.2) (layer "F.Cu") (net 5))
 (segment (start 150.9 71.6) (end 150.9 71.4) (width 0.2) (layer "F.Cu") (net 5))
 (segment (start 151.4 74.1) (end 151.9 73.6) (width 0.2) (layer "F.Cu") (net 5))
 (segment (start 151.9 73.6) (end 151.9 72.6) (width 0.2) (layer "F.Cu") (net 5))
 (segment (start 151.4 74.45) (end 151.225 74.275) (width 0.2) (layer "F.Cu") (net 5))
 (segment (start 149.075 70.265) (end 149.765 70.265) (width 0.2) (layer "F.Cu") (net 5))
 (segment (start 149.765 70.265) (end 150.9 71.4) (width 0.2) (layer "F.Cu") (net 5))
 (segment (start 151.4 75.540001) (end 151.4 74.1) (width 0.2) (layer "F.Cu") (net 5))
 (segment (start 151.225 74.275) (end 151.4 74.1) (width 0.2) (layer "F.Cu") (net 5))
 (segment (start 148.2 74.275) (end 151.225 74.275) (width 0.2) (layer "F.Cu") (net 5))
 (segment (start 151.9 72.6) (end 150.9 71.6) (width 0.2) (layer "F.Cu") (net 5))
 (segment (start 142.025 65.775) (end 141.4 66.4) (width 0.2) (layer "F.Cu") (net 2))
 (segment (start 143.975 65.85) (end 143.9 65.775) (width 0.2) (layer "F.Cu") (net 2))
 (segment (start 143.9 65.775) (end 142.025 65.775) (width 0.2) (layer "F.Cu") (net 2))
 (segment (start 147.5375 65.85) (end 143.975 65.85) (width 0.2) (layer "F.Cu") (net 2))
 (segment (start 141.4 66.4) (end 151.8 66.4) (width 1) (layer "B.Cu") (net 2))
 (segment (start 151.9 69.04) (end 151.8 68.94) (width 0.5) (layer "F.Cu") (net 7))
 (segment (start 151.9 71.162499) (end 151.9 69.04) (width 0.5) (layer "F.Cu") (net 7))
 (segment (start 145.175 74.125) (end 145.9 73.4) (width 0.2) (layer "F.Cu") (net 9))
 (segment (start 145.175 74.4) (end 145.175 74.125) (width 0.2) (layer "F.Cu") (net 9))
 (segment (start 144.795 68.995) (end 145.9 70.1) (width 0.2) (layer "F.Cu") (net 9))
 (segment (start 145.9 73.4) (end 145.9 70.1) (width 0.2) (layer "F.Cu") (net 9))
 (segment (start 145.175 75.9) (end 145.175 74.4) (width 0.2) (layer "F.Cu") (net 9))
 (segment (start 144.125 68.995) (end 144.795 68.995) (width 0.2) (layer "F.Cu") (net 9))
 (segment (start 143.925 73.975) (end 144.4 73.5) (width 0.2) (layer "F.Cu") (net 8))
 (segment (start 145.4 72.1) (end 144.835 71.535) (width 0.2) (layer "F.Cu") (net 8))
 (segment (start 145.4 73.3) (end 145.4 72.1) (width 0.2) (layer "F.Cu") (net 8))
 (segment (start 143.925 74.4) (end 143.925 73.975) (width 0.2) (layer "F.Cu") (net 8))
 (segment (start 143.925 75.9) (end 143.925 74.4) (width 0.2) (layer "F.Cu") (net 8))
 (segment (start 144.835 71.535) (end 144.125 71.535) (width 0.2) (layer "F.Cu") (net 8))
 (segment (start 144.4 73.5) (end 145.2 73.5) (width 0.2) (layer "F.Cu") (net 8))
 (segment (start 145.2 73.5) (end 145.4 73.3) (width 0.2) (layer "F.Cu") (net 8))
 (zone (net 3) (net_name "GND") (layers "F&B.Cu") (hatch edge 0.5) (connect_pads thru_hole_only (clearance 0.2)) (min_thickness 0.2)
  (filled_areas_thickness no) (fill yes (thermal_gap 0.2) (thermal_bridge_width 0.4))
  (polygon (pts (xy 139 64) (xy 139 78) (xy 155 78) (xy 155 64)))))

